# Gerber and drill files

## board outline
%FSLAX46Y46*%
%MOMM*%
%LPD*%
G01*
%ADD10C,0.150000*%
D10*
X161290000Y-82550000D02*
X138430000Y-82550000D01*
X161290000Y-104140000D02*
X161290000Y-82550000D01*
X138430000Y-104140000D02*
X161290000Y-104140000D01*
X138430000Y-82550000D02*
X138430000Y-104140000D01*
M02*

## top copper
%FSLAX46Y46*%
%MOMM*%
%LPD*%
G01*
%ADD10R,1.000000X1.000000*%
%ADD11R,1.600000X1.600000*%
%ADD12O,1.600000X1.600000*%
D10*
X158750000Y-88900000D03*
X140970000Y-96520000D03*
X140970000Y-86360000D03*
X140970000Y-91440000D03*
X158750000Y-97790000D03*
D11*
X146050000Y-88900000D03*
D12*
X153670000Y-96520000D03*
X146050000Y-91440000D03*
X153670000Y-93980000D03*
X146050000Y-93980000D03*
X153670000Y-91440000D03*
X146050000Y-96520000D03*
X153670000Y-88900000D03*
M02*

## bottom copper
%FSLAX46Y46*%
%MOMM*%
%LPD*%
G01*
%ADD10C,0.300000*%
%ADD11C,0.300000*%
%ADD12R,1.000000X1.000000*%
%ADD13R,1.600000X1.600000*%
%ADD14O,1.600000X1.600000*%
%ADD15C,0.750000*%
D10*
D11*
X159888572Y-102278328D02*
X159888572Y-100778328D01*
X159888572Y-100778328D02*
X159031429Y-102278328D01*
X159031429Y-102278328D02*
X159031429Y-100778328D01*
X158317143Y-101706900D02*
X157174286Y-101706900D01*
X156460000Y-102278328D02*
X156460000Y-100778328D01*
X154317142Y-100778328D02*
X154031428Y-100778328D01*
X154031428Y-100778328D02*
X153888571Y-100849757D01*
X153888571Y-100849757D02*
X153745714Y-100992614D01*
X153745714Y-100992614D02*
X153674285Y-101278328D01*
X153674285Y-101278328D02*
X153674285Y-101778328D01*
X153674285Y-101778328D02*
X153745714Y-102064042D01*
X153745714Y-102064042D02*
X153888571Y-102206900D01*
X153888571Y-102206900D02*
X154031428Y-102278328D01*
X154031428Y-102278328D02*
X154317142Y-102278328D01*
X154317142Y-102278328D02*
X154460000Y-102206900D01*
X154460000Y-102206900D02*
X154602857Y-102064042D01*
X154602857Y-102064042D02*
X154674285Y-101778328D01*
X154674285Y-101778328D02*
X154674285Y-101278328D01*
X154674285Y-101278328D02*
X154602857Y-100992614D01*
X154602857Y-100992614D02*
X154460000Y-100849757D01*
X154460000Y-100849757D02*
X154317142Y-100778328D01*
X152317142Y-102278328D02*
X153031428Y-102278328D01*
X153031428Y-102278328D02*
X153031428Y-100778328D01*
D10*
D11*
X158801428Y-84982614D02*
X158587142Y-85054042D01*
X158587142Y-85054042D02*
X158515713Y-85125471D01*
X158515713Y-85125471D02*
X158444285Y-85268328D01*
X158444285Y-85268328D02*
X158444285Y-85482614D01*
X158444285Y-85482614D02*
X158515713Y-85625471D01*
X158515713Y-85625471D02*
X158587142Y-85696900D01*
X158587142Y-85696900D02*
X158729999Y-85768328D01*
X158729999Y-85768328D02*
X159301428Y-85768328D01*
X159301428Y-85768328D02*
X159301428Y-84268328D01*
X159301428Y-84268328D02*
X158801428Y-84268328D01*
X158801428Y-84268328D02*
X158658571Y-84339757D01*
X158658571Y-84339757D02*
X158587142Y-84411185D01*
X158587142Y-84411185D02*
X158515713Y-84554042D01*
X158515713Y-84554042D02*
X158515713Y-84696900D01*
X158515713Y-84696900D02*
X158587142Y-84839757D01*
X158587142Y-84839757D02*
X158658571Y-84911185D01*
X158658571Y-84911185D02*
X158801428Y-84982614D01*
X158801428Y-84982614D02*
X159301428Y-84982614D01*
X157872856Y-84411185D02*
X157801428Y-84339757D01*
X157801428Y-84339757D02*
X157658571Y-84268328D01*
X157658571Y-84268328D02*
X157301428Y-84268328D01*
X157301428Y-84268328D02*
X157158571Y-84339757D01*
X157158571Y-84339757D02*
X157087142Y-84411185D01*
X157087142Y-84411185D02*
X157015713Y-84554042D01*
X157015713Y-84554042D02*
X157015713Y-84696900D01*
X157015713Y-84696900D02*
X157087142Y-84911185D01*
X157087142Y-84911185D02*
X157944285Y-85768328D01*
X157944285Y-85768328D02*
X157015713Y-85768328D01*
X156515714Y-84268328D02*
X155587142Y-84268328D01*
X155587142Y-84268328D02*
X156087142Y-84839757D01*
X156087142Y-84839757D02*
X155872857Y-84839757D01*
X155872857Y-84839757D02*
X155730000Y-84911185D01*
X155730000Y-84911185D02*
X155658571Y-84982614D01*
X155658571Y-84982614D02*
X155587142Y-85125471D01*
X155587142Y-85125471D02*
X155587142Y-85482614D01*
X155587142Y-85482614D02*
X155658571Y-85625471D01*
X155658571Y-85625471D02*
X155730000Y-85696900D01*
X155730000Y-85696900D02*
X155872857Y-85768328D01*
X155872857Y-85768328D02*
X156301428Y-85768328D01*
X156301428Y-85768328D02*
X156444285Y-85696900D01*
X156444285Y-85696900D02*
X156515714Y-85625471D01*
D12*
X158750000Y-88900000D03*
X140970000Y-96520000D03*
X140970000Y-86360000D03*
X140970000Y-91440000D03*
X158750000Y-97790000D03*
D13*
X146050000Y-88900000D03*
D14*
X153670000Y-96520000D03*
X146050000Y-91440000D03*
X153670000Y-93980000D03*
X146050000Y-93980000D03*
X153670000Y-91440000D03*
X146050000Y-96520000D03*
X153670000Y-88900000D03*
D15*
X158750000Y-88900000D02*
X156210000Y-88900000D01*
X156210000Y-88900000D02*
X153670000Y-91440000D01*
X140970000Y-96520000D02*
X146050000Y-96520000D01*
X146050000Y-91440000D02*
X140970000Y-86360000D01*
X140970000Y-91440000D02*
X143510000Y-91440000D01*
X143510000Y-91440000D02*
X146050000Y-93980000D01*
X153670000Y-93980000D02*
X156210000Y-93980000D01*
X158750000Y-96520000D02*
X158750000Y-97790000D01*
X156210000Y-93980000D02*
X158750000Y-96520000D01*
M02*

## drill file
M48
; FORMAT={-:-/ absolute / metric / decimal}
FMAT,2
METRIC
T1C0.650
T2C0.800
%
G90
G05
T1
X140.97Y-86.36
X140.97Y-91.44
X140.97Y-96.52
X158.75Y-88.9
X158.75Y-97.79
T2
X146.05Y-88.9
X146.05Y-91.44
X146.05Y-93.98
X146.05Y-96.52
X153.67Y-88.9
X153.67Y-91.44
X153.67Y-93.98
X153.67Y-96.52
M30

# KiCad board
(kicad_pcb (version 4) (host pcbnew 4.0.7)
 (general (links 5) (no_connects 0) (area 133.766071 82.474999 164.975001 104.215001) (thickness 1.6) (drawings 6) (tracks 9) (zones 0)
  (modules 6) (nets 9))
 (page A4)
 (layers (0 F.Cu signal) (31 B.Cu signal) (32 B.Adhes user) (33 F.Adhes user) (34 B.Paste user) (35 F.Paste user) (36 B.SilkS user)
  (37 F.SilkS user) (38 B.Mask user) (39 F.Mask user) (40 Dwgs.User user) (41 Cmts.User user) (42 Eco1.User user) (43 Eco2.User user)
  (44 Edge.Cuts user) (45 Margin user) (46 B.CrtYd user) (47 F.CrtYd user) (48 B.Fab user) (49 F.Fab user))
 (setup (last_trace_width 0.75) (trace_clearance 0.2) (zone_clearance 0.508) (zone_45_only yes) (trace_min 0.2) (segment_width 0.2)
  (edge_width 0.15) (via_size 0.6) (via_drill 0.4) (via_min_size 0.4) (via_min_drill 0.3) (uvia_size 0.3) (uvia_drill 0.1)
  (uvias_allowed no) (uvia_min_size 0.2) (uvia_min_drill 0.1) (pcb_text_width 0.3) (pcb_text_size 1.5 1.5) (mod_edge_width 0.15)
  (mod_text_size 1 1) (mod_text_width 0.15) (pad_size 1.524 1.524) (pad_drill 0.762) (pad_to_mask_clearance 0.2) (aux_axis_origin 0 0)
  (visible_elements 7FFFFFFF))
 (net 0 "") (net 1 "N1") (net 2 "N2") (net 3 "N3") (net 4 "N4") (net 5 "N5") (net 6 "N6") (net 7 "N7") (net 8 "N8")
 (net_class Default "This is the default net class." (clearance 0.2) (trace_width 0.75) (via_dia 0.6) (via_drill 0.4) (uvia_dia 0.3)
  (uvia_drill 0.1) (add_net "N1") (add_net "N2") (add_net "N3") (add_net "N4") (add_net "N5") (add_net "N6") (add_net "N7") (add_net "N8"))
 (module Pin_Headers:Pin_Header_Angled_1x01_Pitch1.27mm (layer F.Cu) (at 158.75 88.9)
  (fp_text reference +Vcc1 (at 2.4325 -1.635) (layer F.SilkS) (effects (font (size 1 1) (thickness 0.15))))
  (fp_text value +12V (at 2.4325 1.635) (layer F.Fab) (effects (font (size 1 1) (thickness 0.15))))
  (pad 1 thru_hole rect (at 0 0) (size 1 1) (drill 0.65) (layers *.Cu *.Mask) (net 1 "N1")))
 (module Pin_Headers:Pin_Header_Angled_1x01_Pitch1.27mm (layer F.Cu) (at 140.97 96.52 180)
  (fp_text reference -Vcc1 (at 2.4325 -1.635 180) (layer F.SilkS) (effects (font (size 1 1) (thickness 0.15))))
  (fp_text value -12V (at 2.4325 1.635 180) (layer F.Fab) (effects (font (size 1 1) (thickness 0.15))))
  (pad 1 thru_hole rect (at 0 0 180) (size 1 1) (drill 0.65) (layers *.Cu *.Mask) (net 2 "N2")))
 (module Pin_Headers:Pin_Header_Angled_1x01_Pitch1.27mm (layer F.Cu) (at 140.97 86.36 180)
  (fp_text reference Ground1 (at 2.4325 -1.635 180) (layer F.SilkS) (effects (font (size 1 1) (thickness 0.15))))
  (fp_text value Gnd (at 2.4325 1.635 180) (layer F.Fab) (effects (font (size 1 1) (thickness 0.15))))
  (pad 1 thru_hole rect (at 0 0 180) (size 1 1) (drill 0.65) (layers *.Cu *.Mask) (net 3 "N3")))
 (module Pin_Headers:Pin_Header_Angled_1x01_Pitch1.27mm (layer F.Cu) (at 140.97 91.44 180)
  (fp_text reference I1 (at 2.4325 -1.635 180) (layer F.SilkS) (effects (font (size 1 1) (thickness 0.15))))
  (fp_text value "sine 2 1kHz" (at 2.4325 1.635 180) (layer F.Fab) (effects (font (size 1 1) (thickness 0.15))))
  (pad 1 thru_hole rect (at 0 0 180) (size 1 1) (drill 0.65) (layers *.Cu *.Mask) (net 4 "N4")))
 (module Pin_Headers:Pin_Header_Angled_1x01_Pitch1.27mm (layer F.Cu) (at 158.75 97.79)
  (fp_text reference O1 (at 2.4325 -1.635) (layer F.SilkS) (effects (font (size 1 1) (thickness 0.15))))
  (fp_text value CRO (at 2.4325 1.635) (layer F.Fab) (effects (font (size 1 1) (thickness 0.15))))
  (pad 1 thru_hole rect (at 0 0) (size 1 1) (drill 0.65) (layers *.Cu *.Mask) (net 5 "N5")))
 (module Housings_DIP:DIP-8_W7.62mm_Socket (layer F.Cu) (at 146.05 88.9)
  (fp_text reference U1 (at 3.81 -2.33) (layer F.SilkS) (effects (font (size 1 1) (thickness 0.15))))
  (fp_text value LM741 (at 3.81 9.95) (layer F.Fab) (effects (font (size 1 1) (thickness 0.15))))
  (pad 1 thru_hole rect (at 0 0) (size 1.6 1.6) (drill 0.8) (layers *.Cu *.Mask) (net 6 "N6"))
  (pad 5 thru_hole oval (at 7.62 7.62) (size 1.6 1.6) (drill 0.8) (layers *.Cu *.Mask) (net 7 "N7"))
  (pad 2 thru_hole oval (at 0 2.54) (size 1.6 1.6) (drill 0.8) (layers *.Cu *.Mask) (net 3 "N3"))
  (pad 6 thru_hole oval (at 7.62 5.08) (size 1.6 1.6) (drill 0.8) (layers *.Cu *.Mask) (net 5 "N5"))
  (pad 3 thru_hole oval (at 0 5.08) (size 1.6 1.6) (drill 0.8) (layers *.Cu *.Mask) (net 4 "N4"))
  (pad 7 thru_hole oval (at 7.62 2.54) (size 1.6 1.6) (drill 0.8) (layers *.Cu *.Mask) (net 1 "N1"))
  (pad 4 thru_hole oval (at 0 7.62) (size 1.6 1.6) (drill 0.8) (layers *.Cu *.Mask) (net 2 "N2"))
  (pad 8 thru_hole oval (at 7.62 0) (size 1.6 1.6) (drill 0.8) (layers *.Cu *.Mask) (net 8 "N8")))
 (gr_line (start 161.29 82.55) (end 138.43 82.55) (angle 90) (layer Edge.Cuts) (width 0.15))
 (gr_line (start 161.29 104.14) (end 161.29 82.55) (angle 90) (layer Edge.Cuts) (width 0.15))
 (gr_line (start 138.43 104.14) (end 161.29 104.14) (angle 90) (layer Edge.Cuts) (width 0.15))
 (gr_line (start 138.43 82.55) (end 138.43 104.14) (angle 90) (layer Edge.Cuts) (width 0.15))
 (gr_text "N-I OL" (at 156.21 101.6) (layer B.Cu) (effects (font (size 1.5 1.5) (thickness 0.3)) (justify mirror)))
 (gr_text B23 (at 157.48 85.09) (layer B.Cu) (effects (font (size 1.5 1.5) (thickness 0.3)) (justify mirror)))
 (segment (start 158.75 88.9) (end 156.21 88.9) (width 0.75) (layer B.Cu) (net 1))
 (segment (start 156.21 88.9) (end 153.67 91.44) (width 0.75) (layer B.Cu) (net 1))
 (segment (start 140.97 96.52) (end 146.05 96.52) (width 0.75) (layer B.Cu) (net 2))
 (segment (start 146.05 91.44) (end 140.97 86.36) (width 0.75) (layer B.Cu) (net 3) (status C00000))
 (segment (start 140.97 91.44) (end 143.51 91.44) (width 0.75) (layer B.Cu) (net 4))
 (segment (start 143.51 91.44) (end 146.05 93.98) (width 0.75) (layer B.Cu) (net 4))
 (segment (start 153.67 93.98) (end 156.21 93.98) (width 0.75) (layer B.Cu) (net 5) (status 400000))
 (segment (start 158.75 96.52) (end 158.75 97.79) (width 0.75) (layer B.Cu) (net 5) (status 800000))
 (segment (start 156.21 93.98) (end 158.75 96.52) (width 0.75) (layer B.Cu) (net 5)))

